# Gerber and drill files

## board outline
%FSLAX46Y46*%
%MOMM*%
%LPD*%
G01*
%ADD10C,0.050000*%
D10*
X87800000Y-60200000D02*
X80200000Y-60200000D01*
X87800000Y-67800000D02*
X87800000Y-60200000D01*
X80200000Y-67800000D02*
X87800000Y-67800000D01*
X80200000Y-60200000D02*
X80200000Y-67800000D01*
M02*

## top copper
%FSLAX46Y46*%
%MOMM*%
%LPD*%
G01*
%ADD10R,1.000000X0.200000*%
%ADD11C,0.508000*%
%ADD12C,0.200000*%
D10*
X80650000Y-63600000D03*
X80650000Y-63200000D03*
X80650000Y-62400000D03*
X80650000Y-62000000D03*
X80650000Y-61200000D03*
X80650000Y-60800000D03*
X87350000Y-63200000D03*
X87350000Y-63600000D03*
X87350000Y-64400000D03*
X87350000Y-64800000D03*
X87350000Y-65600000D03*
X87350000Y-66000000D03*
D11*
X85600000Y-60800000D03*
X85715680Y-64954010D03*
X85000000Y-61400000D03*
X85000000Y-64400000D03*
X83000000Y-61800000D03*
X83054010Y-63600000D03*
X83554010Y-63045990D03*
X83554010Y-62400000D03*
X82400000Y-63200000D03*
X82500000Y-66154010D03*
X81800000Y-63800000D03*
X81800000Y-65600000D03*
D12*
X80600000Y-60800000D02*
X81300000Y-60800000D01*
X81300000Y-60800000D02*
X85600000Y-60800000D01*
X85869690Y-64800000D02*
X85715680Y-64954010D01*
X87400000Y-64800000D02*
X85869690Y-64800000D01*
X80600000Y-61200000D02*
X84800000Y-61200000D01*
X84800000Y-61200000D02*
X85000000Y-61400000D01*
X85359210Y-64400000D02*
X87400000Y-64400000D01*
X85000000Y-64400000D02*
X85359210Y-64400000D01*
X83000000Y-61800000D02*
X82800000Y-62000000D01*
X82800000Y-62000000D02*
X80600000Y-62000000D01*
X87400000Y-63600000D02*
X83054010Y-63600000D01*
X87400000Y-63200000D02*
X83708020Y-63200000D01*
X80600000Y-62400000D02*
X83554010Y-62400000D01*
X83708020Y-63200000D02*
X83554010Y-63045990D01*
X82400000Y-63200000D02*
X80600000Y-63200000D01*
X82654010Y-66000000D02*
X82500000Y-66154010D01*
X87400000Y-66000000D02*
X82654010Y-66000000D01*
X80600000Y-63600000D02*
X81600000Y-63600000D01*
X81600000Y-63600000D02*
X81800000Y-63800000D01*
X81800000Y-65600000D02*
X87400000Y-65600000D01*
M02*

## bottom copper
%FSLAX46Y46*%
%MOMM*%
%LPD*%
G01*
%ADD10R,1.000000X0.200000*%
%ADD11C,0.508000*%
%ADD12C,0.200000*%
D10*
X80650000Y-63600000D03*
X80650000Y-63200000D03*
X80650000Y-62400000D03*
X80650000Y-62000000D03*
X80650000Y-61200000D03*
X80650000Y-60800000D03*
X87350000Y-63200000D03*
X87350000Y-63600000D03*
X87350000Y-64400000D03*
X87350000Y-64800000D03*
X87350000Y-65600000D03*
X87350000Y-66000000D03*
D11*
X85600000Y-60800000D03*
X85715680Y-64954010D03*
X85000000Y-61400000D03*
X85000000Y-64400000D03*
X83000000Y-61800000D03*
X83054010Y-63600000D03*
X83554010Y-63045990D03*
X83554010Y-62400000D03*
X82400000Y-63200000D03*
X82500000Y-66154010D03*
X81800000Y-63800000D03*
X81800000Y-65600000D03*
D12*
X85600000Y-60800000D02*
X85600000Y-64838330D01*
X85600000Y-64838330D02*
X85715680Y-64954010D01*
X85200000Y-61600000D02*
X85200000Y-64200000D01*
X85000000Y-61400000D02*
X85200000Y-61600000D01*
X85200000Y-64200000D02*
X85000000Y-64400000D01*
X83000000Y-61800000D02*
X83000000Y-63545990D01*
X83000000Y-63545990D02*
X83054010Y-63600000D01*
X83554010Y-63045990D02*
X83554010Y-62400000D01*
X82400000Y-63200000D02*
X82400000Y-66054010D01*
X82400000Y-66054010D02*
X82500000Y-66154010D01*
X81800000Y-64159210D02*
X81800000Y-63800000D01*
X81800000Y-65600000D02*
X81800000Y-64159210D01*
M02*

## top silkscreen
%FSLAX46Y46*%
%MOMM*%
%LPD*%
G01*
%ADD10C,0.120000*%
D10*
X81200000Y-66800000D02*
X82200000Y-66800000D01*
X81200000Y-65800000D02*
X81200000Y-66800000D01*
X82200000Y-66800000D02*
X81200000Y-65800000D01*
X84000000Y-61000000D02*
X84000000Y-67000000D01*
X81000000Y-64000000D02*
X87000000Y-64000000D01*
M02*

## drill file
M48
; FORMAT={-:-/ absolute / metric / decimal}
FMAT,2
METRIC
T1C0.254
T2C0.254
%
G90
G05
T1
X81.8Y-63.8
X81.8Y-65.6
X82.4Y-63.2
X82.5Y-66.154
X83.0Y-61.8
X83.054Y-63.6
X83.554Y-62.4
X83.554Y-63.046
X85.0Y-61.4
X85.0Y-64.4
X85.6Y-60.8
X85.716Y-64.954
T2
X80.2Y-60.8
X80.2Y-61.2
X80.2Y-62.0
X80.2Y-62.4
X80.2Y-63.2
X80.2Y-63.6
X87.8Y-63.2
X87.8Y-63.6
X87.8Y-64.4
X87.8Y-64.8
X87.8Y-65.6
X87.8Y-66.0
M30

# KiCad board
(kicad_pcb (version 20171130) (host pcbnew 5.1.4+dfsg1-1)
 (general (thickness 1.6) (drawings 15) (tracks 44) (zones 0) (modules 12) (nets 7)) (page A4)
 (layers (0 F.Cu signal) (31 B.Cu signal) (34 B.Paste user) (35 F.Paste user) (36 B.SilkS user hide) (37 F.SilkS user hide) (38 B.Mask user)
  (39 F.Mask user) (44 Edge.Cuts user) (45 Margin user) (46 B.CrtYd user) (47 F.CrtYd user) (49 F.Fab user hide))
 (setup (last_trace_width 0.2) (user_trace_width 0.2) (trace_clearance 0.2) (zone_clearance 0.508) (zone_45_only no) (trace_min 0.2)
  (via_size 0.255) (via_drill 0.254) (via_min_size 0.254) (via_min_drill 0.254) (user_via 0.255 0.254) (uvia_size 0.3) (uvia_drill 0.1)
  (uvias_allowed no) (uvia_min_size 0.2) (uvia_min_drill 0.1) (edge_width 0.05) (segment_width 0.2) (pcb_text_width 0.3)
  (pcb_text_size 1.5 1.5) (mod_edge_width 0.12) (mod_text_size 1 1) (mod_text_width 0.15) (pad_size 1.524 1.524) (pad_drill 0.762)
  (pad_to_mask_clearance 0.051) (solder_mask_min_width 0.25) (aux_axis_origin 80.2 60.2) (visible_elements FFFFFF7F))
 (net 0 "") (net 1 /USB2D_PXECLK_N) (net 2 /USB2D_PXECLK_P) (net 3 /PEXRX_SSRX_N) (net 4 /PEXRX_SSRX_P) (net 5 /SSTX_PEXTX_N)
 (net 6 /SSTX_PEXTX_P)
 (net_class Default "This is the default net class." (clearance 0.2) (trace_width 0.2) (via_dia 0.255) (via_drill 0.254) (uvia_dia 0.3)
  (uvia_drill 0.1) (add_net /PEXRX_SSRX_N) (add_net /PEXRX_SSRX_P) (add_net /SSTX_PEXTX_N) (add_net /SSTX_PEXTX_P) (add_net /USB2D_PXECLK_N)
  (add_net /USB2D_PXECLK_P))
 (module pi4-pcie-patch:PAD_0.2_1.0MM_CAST (layer F.Cu) (at 80.2 63.6)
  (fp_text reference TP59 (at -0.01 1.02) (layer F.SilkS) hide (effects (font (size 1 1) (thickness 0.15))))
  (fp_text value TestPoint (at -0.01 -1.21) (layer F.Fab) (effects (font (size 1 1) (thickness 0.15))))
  (pad 1 thru_hole rect (at 0 0) (size 1 0.2) (drill 0.254 (offset 0.45 0)) (layers *.Cu *.Mask) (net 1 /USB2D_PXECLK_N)))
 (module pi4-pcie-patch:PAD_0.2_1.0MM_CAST (layer F.Cu) (at 80.2 63.2)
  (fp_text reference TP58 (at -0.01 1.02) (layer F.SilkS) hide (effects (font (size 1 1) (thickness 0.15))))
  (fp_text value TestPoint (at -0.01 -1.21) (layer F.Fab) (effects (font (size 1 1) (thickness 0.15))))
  (pad 1 thru_hole rect (at 0 0) (size 1 0.2) (drill 0.254 (offset 0.45 0)) (layers *.Cu *.Mask) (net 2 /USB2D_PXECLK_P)))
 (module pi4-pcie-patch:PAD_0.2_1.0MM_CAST (layer F.Cu) (at 80.2 62.4)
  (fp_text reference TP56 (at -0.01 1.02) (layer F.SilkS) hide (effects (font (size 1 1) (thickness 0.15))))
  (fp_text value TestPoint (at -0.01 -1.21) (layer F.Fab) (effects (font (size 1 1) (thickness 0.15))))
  (pad 1 thru_hole rect (at 0 0) (size 1 0.2) (drill 0.254 (offset 0.45 0)) (layers *.Cu *.Mask) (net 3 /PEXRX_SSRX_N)))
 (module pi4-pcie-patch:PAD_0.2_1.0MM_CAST (layer F.Cu) (at 80.2 62)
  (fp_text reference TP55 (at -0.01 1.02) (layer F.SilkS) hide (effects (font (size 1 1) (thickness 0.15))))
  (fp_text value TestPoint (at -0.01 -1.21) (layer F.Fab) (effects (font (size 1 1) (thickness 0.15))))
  (pad 1 thru_hole rect (at 0 0) (size 1 0.2) (drill 0.254 (offset 0.45 0)) (layers *.Cu *.Mask) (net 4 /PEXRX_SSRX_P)))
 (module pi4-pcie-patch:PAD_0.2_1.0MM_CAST (layer F.Cu) (at 80.2 61.2)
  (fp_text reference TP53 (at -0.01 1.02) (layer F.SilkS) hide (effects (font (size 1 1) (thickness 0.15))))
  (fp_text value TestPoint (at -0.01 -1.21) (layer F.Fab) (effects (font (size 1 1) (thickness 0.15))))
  (pad 1 thru_hole rect (at 0 0) (size 1 0.2) (drill 0.254 (offset 0.45 0)) (layers *.Cu *.Mask) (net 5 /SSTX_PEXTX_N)))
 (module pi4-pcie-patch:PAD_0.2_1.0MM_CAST (layer F.Cu) (at 80.2 60.8)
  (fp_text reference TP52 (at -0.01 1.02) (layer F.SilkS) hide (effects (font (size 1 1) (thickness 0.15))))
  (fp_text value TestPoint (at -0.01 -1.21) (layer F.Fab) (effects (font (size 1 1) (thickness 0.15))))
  (pad 1 thru_hole rect (at 0 0) (size 1 0.2) (drill 0.254 (offset 0.45 0)) (layers *.Cu *.Mask) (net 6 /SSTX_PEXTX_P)))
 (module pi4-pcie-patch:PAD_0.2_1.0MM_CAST (layer F.Cu) (at 87.8 63.2 180)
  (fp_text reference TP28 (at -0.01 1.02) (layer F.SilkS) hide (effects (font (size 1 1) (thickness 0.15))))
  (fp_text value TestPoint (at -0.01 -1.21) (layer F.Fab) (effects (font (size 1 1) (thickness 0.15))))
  (pad 1 thru_hole rect (at 0 0 180) (size 1 0.2) (drill 0.254 (offset 0.45 0)) (layers *.Cu *.Mask) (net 3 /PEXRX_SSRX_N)))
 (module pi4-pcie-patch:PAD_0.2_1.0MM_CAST (layer F.Cu) (at 87.8 63.6 180)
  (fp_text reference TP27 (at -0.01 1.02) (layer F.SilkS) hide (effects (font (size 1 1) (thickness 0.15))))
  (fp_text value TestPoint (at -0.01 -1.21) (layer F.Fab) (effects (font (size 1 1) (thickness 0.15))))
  (pad 1 thru_hole rect (at 0 0 180) (size 1 0.2) (drill 0.254 (offset 0.45 0)) (layers *.Cu *.Mask) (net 4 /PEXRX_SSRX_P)))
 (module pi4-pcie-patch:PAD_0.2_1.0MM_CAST (layer F.Cu) (at 87.8 64.4 180)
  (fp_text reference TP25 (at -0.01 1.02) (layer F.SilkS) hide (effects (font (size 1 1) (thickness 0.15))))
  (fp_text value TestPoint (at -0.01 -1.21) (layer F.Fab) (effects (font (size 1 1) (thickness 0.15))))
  (pad 1 thru_hole rect (at 0 0 180) (size 1 0.2) (drill 0.254 (offset 0.45 0)) (layers *.Cu *.Mask) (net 5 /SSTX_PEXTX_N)))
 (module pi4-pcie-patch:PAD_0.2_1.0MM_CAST (layer F.Cu) (at 87.8 64.8 180)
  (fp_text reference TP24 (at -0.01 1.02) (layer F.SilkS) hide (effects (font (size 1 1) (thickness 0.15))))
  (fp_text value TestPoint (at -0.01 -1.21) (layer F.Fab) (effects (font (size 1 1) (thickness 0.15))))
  (pad 1 thru_hole rect (at 0 0 180) (size 1 0.2) (drill 0.254 (offset 0.45 0)) (layers *.Cu *.Mask) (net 6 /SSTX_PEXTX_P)))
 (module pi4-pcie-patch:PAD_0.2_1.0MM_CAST (layer F.Cu) (at 87.8 65.6 180)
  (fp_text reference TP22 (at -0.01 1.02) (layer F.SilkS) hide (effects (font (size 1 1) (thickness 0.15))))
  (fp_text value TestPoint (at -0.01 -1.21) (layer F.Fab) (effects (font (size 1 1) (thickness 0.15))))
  (pad 1 thru_hole rect (at 0 0 180) (size 1 0.2) (drill 0.254 (offset 0.45 0)) (layers *.Cu *.Mask) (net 1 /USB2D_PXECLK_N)))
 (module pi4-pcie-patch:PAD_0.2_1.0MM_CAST (layer F.Cu) (at 87.8 66 180)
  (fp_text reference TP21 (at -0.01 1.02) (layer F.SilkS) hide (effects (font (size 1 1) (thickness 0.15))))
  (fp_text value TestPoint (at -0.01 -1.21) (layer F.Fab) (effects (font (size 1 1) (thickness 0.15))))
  (pad 1 thru_hole rect (at 0 0 180) (size 1 0.2) (drill 0.254 (offset 0.45 0)) (layers *.Cu *.Mask) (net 2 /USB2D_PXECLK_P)))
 (gr_line (start 81.2 66.8) (end 82.2 66.8) (layer F.SilkS) (width 0.12))
 (gr_line (start 81.2 65.8) (end 81.2 66.8) (layer F.SilkS) (width 0.12))
 (gr_line (start 82.2 66.8) (end 81.2 65.8) (layer F.SilkS) (width 0.12))
 (gr_line (start 84 61) (end 84 67) (layer F.SilkS) (width 0.12))
 (gr_line (start 81 64) (end 87 64) (layer F.SilkS) (width 0.12))
 (gr_line (start 87.8 60.2) (end 80.2 60.2) (layer Edge.Cuts) (width 0.05))
 (gr_line (start 87.8 67.8) (end 87.8 60.2) (layer Edge.Cuts) (width 0.05))
 (gr_line (start 80.2 67.8) (end 87.8 67.8) (layer Edge.Cuts) (width 0.05))
 (gr_line (start 80.2 60.2) (end 80.2 67.8) (layer Edge.Cuts) (width 0.05))
 (segment (start 80.6 60.8) (end 81.3 60.8) (width 0.2) (layer F.Cu) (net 6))
 (via (at 85.6 60.8) (size 0.508) (drill 0.254) (layers F.Cu B.Cu) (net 6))
 (segment (start 81.3 60.8) (end 85.6 60.8) (width 0.2) (layer F.Cu) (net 6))
 (segment (start 85.6 60.8) (end 85.6 64.83833) (width 0.2) (layer B.Cu) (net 6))
 (segment (start 85.86969 64.8) (end 85.71568 64.95401) (width 0.2) (layer F.Cu) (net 6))
 (via (at 85.71568 64.95401) (size 0.508) (drill 0.254) (layers F.Cu B.Cu) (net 6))
 (segment (start 87.4 64.8) (end 85.86969 64.8) (width 0.2) (layer F.Cu) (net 6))
 (segment (start 85.6 64.83833) (end 85.71568 64.95401) (width 0.2) (layer B.Cu) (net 6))
 (via (at 85 61.4) (size 0.508) (drill 0.254) (layers F.Cu B.Cu) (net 5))
 (segment (start 80.6 61.2) (end 84.8 61.2) (width 0.2) (layer F.Cu) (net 5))
 (segment (start 84.8 61.2) (end 85 61.4) (width 0.2) (layer F.Cu) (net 5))
 (segment (start 85.2 61.6) (end 85.2 64.2) (width 0.2) (layer B.Cu) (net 5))
 (segment (start 85 61.4) (end 85.2 61.6) (width 0.2) (layer B.Cu) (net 5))
 (via (at 85 64.4) (size 0.508) (drill 0.254) (layers F.Cu B.Cu) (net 5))
 (segment (start 85.2 64.2) (end 85 64.4) (width 0.2) (layer B.Cu) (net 5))
 (segment (start 85.35921 64.4) (end 87.4 64.4) (width 0.2) (layer F.Cu) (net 5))
 (segment (start 85 64.4) (end 85.35921 64.4) (width 0.2) (layer F.Cu) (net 5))
 (via (at 83 61.8) (size 0.508) (drill 0.254) (layers F.Cu B.Cu) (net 4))
 (segment (start 83 61.8) (end 82.8 62) (width 0.2) (layer F.Cu) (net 4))
 (segment (start 82.8 62) (end 80.6 62) (width 0.2) (layer F.Cu) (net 4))
 (segment (start 83 61.8) (end 83 63.54599) (width 0.2) (layer B.Cu) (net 4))
 (segment (start 87.4 63.6) (end 83.05401 63.6) (width 0.2) (layer F.Cu) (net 4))
 (segment (start 83 63.54599) (end 83.05401 63.6) (width 0.2) (layer B.Cu) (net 4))
 (via (at 83.05401 63.6) (size 0.508) (drill 0.254) (layers F.Cu B.Cu) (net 4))
 (via (at 83.55401 63.04599) (size 0.508) (drill 0.254) (layers F.Cu B.Cu) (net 3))
 (segment (start 83.55401 63.04599) (end 83.55401 62.4) (width 0.2) (layer B.Cu) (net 3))
 (segment (start 87.4 63.2) (end 83.70802 63.2) (width 0.2) (layer F.Cu) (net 3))
 (segment (start 80.6 62.4) (end 83.55401 62.4) (width 0.2) (layer F.Cu) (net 3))
 (segment (start 83.70802 63.2) (end 83.55401 63.04599) (width 0.2) (layer F.Cu) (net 3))
 (via (at 83.55401 62.4) (size 0.508) (drill 0.254) (layers F.Cu B.Cu) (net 3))
 (via (at 82.4 63.2) (size 0.508) (drill 0.254) (layers F.Cu B.Cu) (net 2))
 (segment (start 82.4 63.2) (end 80.6 63.2) (width 0.2) (layer F.Cu) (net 2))
 (segment (start 82.4 63.2) (end 82.4 66.05401) (width 0.2) (layer B.Cu) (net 2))
 (segment (start 82.4 66.05401) (end 82.5 66.15401) (width 0.2) (layer B.Cu) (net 2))
 (segment (start 82.65401 66) (end 82.5 66.15401) (width 0.2) (layer F.Cu) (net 2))
 (segment (start 87.4 66) (end 82.65401 66) (width 0.2) (layer F.Cu) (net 2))
 (via (at 82.5 66.15401) (size 0.508) (drill 0.254) (layers F.Cu B.Cu) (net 2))
 (via (at 81.8 63.8) (size 0.508) (drill 0.254) (layers F.Cu B.Cu) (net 1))
 (segment (start 80.6 63.6) (end 81.6 63.6) (width 0.2) (layer F.Cu) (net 1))
 (segment (start 81.6 63.6) (end 81.8 63.8) (width 0.2) (layer F.Cu) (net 1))
 (segment (start 81.8 64.15921) (end 81.8 63.8) (width 0.2) (layer B.Cu) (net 1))
 (segment (start 81.8 65.6) (end 87.4 65.6) (width 0.2) (layer F.Cu) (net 1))
 (via (at 81.8 65.6) (size 0.508) (drill 0.254) (layers F.Cu B.Cu) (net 1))
 (segment (start 81.8 65.6) (end 81.8 64.15921) (width 0.2) (layer B.Cu) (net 1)))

